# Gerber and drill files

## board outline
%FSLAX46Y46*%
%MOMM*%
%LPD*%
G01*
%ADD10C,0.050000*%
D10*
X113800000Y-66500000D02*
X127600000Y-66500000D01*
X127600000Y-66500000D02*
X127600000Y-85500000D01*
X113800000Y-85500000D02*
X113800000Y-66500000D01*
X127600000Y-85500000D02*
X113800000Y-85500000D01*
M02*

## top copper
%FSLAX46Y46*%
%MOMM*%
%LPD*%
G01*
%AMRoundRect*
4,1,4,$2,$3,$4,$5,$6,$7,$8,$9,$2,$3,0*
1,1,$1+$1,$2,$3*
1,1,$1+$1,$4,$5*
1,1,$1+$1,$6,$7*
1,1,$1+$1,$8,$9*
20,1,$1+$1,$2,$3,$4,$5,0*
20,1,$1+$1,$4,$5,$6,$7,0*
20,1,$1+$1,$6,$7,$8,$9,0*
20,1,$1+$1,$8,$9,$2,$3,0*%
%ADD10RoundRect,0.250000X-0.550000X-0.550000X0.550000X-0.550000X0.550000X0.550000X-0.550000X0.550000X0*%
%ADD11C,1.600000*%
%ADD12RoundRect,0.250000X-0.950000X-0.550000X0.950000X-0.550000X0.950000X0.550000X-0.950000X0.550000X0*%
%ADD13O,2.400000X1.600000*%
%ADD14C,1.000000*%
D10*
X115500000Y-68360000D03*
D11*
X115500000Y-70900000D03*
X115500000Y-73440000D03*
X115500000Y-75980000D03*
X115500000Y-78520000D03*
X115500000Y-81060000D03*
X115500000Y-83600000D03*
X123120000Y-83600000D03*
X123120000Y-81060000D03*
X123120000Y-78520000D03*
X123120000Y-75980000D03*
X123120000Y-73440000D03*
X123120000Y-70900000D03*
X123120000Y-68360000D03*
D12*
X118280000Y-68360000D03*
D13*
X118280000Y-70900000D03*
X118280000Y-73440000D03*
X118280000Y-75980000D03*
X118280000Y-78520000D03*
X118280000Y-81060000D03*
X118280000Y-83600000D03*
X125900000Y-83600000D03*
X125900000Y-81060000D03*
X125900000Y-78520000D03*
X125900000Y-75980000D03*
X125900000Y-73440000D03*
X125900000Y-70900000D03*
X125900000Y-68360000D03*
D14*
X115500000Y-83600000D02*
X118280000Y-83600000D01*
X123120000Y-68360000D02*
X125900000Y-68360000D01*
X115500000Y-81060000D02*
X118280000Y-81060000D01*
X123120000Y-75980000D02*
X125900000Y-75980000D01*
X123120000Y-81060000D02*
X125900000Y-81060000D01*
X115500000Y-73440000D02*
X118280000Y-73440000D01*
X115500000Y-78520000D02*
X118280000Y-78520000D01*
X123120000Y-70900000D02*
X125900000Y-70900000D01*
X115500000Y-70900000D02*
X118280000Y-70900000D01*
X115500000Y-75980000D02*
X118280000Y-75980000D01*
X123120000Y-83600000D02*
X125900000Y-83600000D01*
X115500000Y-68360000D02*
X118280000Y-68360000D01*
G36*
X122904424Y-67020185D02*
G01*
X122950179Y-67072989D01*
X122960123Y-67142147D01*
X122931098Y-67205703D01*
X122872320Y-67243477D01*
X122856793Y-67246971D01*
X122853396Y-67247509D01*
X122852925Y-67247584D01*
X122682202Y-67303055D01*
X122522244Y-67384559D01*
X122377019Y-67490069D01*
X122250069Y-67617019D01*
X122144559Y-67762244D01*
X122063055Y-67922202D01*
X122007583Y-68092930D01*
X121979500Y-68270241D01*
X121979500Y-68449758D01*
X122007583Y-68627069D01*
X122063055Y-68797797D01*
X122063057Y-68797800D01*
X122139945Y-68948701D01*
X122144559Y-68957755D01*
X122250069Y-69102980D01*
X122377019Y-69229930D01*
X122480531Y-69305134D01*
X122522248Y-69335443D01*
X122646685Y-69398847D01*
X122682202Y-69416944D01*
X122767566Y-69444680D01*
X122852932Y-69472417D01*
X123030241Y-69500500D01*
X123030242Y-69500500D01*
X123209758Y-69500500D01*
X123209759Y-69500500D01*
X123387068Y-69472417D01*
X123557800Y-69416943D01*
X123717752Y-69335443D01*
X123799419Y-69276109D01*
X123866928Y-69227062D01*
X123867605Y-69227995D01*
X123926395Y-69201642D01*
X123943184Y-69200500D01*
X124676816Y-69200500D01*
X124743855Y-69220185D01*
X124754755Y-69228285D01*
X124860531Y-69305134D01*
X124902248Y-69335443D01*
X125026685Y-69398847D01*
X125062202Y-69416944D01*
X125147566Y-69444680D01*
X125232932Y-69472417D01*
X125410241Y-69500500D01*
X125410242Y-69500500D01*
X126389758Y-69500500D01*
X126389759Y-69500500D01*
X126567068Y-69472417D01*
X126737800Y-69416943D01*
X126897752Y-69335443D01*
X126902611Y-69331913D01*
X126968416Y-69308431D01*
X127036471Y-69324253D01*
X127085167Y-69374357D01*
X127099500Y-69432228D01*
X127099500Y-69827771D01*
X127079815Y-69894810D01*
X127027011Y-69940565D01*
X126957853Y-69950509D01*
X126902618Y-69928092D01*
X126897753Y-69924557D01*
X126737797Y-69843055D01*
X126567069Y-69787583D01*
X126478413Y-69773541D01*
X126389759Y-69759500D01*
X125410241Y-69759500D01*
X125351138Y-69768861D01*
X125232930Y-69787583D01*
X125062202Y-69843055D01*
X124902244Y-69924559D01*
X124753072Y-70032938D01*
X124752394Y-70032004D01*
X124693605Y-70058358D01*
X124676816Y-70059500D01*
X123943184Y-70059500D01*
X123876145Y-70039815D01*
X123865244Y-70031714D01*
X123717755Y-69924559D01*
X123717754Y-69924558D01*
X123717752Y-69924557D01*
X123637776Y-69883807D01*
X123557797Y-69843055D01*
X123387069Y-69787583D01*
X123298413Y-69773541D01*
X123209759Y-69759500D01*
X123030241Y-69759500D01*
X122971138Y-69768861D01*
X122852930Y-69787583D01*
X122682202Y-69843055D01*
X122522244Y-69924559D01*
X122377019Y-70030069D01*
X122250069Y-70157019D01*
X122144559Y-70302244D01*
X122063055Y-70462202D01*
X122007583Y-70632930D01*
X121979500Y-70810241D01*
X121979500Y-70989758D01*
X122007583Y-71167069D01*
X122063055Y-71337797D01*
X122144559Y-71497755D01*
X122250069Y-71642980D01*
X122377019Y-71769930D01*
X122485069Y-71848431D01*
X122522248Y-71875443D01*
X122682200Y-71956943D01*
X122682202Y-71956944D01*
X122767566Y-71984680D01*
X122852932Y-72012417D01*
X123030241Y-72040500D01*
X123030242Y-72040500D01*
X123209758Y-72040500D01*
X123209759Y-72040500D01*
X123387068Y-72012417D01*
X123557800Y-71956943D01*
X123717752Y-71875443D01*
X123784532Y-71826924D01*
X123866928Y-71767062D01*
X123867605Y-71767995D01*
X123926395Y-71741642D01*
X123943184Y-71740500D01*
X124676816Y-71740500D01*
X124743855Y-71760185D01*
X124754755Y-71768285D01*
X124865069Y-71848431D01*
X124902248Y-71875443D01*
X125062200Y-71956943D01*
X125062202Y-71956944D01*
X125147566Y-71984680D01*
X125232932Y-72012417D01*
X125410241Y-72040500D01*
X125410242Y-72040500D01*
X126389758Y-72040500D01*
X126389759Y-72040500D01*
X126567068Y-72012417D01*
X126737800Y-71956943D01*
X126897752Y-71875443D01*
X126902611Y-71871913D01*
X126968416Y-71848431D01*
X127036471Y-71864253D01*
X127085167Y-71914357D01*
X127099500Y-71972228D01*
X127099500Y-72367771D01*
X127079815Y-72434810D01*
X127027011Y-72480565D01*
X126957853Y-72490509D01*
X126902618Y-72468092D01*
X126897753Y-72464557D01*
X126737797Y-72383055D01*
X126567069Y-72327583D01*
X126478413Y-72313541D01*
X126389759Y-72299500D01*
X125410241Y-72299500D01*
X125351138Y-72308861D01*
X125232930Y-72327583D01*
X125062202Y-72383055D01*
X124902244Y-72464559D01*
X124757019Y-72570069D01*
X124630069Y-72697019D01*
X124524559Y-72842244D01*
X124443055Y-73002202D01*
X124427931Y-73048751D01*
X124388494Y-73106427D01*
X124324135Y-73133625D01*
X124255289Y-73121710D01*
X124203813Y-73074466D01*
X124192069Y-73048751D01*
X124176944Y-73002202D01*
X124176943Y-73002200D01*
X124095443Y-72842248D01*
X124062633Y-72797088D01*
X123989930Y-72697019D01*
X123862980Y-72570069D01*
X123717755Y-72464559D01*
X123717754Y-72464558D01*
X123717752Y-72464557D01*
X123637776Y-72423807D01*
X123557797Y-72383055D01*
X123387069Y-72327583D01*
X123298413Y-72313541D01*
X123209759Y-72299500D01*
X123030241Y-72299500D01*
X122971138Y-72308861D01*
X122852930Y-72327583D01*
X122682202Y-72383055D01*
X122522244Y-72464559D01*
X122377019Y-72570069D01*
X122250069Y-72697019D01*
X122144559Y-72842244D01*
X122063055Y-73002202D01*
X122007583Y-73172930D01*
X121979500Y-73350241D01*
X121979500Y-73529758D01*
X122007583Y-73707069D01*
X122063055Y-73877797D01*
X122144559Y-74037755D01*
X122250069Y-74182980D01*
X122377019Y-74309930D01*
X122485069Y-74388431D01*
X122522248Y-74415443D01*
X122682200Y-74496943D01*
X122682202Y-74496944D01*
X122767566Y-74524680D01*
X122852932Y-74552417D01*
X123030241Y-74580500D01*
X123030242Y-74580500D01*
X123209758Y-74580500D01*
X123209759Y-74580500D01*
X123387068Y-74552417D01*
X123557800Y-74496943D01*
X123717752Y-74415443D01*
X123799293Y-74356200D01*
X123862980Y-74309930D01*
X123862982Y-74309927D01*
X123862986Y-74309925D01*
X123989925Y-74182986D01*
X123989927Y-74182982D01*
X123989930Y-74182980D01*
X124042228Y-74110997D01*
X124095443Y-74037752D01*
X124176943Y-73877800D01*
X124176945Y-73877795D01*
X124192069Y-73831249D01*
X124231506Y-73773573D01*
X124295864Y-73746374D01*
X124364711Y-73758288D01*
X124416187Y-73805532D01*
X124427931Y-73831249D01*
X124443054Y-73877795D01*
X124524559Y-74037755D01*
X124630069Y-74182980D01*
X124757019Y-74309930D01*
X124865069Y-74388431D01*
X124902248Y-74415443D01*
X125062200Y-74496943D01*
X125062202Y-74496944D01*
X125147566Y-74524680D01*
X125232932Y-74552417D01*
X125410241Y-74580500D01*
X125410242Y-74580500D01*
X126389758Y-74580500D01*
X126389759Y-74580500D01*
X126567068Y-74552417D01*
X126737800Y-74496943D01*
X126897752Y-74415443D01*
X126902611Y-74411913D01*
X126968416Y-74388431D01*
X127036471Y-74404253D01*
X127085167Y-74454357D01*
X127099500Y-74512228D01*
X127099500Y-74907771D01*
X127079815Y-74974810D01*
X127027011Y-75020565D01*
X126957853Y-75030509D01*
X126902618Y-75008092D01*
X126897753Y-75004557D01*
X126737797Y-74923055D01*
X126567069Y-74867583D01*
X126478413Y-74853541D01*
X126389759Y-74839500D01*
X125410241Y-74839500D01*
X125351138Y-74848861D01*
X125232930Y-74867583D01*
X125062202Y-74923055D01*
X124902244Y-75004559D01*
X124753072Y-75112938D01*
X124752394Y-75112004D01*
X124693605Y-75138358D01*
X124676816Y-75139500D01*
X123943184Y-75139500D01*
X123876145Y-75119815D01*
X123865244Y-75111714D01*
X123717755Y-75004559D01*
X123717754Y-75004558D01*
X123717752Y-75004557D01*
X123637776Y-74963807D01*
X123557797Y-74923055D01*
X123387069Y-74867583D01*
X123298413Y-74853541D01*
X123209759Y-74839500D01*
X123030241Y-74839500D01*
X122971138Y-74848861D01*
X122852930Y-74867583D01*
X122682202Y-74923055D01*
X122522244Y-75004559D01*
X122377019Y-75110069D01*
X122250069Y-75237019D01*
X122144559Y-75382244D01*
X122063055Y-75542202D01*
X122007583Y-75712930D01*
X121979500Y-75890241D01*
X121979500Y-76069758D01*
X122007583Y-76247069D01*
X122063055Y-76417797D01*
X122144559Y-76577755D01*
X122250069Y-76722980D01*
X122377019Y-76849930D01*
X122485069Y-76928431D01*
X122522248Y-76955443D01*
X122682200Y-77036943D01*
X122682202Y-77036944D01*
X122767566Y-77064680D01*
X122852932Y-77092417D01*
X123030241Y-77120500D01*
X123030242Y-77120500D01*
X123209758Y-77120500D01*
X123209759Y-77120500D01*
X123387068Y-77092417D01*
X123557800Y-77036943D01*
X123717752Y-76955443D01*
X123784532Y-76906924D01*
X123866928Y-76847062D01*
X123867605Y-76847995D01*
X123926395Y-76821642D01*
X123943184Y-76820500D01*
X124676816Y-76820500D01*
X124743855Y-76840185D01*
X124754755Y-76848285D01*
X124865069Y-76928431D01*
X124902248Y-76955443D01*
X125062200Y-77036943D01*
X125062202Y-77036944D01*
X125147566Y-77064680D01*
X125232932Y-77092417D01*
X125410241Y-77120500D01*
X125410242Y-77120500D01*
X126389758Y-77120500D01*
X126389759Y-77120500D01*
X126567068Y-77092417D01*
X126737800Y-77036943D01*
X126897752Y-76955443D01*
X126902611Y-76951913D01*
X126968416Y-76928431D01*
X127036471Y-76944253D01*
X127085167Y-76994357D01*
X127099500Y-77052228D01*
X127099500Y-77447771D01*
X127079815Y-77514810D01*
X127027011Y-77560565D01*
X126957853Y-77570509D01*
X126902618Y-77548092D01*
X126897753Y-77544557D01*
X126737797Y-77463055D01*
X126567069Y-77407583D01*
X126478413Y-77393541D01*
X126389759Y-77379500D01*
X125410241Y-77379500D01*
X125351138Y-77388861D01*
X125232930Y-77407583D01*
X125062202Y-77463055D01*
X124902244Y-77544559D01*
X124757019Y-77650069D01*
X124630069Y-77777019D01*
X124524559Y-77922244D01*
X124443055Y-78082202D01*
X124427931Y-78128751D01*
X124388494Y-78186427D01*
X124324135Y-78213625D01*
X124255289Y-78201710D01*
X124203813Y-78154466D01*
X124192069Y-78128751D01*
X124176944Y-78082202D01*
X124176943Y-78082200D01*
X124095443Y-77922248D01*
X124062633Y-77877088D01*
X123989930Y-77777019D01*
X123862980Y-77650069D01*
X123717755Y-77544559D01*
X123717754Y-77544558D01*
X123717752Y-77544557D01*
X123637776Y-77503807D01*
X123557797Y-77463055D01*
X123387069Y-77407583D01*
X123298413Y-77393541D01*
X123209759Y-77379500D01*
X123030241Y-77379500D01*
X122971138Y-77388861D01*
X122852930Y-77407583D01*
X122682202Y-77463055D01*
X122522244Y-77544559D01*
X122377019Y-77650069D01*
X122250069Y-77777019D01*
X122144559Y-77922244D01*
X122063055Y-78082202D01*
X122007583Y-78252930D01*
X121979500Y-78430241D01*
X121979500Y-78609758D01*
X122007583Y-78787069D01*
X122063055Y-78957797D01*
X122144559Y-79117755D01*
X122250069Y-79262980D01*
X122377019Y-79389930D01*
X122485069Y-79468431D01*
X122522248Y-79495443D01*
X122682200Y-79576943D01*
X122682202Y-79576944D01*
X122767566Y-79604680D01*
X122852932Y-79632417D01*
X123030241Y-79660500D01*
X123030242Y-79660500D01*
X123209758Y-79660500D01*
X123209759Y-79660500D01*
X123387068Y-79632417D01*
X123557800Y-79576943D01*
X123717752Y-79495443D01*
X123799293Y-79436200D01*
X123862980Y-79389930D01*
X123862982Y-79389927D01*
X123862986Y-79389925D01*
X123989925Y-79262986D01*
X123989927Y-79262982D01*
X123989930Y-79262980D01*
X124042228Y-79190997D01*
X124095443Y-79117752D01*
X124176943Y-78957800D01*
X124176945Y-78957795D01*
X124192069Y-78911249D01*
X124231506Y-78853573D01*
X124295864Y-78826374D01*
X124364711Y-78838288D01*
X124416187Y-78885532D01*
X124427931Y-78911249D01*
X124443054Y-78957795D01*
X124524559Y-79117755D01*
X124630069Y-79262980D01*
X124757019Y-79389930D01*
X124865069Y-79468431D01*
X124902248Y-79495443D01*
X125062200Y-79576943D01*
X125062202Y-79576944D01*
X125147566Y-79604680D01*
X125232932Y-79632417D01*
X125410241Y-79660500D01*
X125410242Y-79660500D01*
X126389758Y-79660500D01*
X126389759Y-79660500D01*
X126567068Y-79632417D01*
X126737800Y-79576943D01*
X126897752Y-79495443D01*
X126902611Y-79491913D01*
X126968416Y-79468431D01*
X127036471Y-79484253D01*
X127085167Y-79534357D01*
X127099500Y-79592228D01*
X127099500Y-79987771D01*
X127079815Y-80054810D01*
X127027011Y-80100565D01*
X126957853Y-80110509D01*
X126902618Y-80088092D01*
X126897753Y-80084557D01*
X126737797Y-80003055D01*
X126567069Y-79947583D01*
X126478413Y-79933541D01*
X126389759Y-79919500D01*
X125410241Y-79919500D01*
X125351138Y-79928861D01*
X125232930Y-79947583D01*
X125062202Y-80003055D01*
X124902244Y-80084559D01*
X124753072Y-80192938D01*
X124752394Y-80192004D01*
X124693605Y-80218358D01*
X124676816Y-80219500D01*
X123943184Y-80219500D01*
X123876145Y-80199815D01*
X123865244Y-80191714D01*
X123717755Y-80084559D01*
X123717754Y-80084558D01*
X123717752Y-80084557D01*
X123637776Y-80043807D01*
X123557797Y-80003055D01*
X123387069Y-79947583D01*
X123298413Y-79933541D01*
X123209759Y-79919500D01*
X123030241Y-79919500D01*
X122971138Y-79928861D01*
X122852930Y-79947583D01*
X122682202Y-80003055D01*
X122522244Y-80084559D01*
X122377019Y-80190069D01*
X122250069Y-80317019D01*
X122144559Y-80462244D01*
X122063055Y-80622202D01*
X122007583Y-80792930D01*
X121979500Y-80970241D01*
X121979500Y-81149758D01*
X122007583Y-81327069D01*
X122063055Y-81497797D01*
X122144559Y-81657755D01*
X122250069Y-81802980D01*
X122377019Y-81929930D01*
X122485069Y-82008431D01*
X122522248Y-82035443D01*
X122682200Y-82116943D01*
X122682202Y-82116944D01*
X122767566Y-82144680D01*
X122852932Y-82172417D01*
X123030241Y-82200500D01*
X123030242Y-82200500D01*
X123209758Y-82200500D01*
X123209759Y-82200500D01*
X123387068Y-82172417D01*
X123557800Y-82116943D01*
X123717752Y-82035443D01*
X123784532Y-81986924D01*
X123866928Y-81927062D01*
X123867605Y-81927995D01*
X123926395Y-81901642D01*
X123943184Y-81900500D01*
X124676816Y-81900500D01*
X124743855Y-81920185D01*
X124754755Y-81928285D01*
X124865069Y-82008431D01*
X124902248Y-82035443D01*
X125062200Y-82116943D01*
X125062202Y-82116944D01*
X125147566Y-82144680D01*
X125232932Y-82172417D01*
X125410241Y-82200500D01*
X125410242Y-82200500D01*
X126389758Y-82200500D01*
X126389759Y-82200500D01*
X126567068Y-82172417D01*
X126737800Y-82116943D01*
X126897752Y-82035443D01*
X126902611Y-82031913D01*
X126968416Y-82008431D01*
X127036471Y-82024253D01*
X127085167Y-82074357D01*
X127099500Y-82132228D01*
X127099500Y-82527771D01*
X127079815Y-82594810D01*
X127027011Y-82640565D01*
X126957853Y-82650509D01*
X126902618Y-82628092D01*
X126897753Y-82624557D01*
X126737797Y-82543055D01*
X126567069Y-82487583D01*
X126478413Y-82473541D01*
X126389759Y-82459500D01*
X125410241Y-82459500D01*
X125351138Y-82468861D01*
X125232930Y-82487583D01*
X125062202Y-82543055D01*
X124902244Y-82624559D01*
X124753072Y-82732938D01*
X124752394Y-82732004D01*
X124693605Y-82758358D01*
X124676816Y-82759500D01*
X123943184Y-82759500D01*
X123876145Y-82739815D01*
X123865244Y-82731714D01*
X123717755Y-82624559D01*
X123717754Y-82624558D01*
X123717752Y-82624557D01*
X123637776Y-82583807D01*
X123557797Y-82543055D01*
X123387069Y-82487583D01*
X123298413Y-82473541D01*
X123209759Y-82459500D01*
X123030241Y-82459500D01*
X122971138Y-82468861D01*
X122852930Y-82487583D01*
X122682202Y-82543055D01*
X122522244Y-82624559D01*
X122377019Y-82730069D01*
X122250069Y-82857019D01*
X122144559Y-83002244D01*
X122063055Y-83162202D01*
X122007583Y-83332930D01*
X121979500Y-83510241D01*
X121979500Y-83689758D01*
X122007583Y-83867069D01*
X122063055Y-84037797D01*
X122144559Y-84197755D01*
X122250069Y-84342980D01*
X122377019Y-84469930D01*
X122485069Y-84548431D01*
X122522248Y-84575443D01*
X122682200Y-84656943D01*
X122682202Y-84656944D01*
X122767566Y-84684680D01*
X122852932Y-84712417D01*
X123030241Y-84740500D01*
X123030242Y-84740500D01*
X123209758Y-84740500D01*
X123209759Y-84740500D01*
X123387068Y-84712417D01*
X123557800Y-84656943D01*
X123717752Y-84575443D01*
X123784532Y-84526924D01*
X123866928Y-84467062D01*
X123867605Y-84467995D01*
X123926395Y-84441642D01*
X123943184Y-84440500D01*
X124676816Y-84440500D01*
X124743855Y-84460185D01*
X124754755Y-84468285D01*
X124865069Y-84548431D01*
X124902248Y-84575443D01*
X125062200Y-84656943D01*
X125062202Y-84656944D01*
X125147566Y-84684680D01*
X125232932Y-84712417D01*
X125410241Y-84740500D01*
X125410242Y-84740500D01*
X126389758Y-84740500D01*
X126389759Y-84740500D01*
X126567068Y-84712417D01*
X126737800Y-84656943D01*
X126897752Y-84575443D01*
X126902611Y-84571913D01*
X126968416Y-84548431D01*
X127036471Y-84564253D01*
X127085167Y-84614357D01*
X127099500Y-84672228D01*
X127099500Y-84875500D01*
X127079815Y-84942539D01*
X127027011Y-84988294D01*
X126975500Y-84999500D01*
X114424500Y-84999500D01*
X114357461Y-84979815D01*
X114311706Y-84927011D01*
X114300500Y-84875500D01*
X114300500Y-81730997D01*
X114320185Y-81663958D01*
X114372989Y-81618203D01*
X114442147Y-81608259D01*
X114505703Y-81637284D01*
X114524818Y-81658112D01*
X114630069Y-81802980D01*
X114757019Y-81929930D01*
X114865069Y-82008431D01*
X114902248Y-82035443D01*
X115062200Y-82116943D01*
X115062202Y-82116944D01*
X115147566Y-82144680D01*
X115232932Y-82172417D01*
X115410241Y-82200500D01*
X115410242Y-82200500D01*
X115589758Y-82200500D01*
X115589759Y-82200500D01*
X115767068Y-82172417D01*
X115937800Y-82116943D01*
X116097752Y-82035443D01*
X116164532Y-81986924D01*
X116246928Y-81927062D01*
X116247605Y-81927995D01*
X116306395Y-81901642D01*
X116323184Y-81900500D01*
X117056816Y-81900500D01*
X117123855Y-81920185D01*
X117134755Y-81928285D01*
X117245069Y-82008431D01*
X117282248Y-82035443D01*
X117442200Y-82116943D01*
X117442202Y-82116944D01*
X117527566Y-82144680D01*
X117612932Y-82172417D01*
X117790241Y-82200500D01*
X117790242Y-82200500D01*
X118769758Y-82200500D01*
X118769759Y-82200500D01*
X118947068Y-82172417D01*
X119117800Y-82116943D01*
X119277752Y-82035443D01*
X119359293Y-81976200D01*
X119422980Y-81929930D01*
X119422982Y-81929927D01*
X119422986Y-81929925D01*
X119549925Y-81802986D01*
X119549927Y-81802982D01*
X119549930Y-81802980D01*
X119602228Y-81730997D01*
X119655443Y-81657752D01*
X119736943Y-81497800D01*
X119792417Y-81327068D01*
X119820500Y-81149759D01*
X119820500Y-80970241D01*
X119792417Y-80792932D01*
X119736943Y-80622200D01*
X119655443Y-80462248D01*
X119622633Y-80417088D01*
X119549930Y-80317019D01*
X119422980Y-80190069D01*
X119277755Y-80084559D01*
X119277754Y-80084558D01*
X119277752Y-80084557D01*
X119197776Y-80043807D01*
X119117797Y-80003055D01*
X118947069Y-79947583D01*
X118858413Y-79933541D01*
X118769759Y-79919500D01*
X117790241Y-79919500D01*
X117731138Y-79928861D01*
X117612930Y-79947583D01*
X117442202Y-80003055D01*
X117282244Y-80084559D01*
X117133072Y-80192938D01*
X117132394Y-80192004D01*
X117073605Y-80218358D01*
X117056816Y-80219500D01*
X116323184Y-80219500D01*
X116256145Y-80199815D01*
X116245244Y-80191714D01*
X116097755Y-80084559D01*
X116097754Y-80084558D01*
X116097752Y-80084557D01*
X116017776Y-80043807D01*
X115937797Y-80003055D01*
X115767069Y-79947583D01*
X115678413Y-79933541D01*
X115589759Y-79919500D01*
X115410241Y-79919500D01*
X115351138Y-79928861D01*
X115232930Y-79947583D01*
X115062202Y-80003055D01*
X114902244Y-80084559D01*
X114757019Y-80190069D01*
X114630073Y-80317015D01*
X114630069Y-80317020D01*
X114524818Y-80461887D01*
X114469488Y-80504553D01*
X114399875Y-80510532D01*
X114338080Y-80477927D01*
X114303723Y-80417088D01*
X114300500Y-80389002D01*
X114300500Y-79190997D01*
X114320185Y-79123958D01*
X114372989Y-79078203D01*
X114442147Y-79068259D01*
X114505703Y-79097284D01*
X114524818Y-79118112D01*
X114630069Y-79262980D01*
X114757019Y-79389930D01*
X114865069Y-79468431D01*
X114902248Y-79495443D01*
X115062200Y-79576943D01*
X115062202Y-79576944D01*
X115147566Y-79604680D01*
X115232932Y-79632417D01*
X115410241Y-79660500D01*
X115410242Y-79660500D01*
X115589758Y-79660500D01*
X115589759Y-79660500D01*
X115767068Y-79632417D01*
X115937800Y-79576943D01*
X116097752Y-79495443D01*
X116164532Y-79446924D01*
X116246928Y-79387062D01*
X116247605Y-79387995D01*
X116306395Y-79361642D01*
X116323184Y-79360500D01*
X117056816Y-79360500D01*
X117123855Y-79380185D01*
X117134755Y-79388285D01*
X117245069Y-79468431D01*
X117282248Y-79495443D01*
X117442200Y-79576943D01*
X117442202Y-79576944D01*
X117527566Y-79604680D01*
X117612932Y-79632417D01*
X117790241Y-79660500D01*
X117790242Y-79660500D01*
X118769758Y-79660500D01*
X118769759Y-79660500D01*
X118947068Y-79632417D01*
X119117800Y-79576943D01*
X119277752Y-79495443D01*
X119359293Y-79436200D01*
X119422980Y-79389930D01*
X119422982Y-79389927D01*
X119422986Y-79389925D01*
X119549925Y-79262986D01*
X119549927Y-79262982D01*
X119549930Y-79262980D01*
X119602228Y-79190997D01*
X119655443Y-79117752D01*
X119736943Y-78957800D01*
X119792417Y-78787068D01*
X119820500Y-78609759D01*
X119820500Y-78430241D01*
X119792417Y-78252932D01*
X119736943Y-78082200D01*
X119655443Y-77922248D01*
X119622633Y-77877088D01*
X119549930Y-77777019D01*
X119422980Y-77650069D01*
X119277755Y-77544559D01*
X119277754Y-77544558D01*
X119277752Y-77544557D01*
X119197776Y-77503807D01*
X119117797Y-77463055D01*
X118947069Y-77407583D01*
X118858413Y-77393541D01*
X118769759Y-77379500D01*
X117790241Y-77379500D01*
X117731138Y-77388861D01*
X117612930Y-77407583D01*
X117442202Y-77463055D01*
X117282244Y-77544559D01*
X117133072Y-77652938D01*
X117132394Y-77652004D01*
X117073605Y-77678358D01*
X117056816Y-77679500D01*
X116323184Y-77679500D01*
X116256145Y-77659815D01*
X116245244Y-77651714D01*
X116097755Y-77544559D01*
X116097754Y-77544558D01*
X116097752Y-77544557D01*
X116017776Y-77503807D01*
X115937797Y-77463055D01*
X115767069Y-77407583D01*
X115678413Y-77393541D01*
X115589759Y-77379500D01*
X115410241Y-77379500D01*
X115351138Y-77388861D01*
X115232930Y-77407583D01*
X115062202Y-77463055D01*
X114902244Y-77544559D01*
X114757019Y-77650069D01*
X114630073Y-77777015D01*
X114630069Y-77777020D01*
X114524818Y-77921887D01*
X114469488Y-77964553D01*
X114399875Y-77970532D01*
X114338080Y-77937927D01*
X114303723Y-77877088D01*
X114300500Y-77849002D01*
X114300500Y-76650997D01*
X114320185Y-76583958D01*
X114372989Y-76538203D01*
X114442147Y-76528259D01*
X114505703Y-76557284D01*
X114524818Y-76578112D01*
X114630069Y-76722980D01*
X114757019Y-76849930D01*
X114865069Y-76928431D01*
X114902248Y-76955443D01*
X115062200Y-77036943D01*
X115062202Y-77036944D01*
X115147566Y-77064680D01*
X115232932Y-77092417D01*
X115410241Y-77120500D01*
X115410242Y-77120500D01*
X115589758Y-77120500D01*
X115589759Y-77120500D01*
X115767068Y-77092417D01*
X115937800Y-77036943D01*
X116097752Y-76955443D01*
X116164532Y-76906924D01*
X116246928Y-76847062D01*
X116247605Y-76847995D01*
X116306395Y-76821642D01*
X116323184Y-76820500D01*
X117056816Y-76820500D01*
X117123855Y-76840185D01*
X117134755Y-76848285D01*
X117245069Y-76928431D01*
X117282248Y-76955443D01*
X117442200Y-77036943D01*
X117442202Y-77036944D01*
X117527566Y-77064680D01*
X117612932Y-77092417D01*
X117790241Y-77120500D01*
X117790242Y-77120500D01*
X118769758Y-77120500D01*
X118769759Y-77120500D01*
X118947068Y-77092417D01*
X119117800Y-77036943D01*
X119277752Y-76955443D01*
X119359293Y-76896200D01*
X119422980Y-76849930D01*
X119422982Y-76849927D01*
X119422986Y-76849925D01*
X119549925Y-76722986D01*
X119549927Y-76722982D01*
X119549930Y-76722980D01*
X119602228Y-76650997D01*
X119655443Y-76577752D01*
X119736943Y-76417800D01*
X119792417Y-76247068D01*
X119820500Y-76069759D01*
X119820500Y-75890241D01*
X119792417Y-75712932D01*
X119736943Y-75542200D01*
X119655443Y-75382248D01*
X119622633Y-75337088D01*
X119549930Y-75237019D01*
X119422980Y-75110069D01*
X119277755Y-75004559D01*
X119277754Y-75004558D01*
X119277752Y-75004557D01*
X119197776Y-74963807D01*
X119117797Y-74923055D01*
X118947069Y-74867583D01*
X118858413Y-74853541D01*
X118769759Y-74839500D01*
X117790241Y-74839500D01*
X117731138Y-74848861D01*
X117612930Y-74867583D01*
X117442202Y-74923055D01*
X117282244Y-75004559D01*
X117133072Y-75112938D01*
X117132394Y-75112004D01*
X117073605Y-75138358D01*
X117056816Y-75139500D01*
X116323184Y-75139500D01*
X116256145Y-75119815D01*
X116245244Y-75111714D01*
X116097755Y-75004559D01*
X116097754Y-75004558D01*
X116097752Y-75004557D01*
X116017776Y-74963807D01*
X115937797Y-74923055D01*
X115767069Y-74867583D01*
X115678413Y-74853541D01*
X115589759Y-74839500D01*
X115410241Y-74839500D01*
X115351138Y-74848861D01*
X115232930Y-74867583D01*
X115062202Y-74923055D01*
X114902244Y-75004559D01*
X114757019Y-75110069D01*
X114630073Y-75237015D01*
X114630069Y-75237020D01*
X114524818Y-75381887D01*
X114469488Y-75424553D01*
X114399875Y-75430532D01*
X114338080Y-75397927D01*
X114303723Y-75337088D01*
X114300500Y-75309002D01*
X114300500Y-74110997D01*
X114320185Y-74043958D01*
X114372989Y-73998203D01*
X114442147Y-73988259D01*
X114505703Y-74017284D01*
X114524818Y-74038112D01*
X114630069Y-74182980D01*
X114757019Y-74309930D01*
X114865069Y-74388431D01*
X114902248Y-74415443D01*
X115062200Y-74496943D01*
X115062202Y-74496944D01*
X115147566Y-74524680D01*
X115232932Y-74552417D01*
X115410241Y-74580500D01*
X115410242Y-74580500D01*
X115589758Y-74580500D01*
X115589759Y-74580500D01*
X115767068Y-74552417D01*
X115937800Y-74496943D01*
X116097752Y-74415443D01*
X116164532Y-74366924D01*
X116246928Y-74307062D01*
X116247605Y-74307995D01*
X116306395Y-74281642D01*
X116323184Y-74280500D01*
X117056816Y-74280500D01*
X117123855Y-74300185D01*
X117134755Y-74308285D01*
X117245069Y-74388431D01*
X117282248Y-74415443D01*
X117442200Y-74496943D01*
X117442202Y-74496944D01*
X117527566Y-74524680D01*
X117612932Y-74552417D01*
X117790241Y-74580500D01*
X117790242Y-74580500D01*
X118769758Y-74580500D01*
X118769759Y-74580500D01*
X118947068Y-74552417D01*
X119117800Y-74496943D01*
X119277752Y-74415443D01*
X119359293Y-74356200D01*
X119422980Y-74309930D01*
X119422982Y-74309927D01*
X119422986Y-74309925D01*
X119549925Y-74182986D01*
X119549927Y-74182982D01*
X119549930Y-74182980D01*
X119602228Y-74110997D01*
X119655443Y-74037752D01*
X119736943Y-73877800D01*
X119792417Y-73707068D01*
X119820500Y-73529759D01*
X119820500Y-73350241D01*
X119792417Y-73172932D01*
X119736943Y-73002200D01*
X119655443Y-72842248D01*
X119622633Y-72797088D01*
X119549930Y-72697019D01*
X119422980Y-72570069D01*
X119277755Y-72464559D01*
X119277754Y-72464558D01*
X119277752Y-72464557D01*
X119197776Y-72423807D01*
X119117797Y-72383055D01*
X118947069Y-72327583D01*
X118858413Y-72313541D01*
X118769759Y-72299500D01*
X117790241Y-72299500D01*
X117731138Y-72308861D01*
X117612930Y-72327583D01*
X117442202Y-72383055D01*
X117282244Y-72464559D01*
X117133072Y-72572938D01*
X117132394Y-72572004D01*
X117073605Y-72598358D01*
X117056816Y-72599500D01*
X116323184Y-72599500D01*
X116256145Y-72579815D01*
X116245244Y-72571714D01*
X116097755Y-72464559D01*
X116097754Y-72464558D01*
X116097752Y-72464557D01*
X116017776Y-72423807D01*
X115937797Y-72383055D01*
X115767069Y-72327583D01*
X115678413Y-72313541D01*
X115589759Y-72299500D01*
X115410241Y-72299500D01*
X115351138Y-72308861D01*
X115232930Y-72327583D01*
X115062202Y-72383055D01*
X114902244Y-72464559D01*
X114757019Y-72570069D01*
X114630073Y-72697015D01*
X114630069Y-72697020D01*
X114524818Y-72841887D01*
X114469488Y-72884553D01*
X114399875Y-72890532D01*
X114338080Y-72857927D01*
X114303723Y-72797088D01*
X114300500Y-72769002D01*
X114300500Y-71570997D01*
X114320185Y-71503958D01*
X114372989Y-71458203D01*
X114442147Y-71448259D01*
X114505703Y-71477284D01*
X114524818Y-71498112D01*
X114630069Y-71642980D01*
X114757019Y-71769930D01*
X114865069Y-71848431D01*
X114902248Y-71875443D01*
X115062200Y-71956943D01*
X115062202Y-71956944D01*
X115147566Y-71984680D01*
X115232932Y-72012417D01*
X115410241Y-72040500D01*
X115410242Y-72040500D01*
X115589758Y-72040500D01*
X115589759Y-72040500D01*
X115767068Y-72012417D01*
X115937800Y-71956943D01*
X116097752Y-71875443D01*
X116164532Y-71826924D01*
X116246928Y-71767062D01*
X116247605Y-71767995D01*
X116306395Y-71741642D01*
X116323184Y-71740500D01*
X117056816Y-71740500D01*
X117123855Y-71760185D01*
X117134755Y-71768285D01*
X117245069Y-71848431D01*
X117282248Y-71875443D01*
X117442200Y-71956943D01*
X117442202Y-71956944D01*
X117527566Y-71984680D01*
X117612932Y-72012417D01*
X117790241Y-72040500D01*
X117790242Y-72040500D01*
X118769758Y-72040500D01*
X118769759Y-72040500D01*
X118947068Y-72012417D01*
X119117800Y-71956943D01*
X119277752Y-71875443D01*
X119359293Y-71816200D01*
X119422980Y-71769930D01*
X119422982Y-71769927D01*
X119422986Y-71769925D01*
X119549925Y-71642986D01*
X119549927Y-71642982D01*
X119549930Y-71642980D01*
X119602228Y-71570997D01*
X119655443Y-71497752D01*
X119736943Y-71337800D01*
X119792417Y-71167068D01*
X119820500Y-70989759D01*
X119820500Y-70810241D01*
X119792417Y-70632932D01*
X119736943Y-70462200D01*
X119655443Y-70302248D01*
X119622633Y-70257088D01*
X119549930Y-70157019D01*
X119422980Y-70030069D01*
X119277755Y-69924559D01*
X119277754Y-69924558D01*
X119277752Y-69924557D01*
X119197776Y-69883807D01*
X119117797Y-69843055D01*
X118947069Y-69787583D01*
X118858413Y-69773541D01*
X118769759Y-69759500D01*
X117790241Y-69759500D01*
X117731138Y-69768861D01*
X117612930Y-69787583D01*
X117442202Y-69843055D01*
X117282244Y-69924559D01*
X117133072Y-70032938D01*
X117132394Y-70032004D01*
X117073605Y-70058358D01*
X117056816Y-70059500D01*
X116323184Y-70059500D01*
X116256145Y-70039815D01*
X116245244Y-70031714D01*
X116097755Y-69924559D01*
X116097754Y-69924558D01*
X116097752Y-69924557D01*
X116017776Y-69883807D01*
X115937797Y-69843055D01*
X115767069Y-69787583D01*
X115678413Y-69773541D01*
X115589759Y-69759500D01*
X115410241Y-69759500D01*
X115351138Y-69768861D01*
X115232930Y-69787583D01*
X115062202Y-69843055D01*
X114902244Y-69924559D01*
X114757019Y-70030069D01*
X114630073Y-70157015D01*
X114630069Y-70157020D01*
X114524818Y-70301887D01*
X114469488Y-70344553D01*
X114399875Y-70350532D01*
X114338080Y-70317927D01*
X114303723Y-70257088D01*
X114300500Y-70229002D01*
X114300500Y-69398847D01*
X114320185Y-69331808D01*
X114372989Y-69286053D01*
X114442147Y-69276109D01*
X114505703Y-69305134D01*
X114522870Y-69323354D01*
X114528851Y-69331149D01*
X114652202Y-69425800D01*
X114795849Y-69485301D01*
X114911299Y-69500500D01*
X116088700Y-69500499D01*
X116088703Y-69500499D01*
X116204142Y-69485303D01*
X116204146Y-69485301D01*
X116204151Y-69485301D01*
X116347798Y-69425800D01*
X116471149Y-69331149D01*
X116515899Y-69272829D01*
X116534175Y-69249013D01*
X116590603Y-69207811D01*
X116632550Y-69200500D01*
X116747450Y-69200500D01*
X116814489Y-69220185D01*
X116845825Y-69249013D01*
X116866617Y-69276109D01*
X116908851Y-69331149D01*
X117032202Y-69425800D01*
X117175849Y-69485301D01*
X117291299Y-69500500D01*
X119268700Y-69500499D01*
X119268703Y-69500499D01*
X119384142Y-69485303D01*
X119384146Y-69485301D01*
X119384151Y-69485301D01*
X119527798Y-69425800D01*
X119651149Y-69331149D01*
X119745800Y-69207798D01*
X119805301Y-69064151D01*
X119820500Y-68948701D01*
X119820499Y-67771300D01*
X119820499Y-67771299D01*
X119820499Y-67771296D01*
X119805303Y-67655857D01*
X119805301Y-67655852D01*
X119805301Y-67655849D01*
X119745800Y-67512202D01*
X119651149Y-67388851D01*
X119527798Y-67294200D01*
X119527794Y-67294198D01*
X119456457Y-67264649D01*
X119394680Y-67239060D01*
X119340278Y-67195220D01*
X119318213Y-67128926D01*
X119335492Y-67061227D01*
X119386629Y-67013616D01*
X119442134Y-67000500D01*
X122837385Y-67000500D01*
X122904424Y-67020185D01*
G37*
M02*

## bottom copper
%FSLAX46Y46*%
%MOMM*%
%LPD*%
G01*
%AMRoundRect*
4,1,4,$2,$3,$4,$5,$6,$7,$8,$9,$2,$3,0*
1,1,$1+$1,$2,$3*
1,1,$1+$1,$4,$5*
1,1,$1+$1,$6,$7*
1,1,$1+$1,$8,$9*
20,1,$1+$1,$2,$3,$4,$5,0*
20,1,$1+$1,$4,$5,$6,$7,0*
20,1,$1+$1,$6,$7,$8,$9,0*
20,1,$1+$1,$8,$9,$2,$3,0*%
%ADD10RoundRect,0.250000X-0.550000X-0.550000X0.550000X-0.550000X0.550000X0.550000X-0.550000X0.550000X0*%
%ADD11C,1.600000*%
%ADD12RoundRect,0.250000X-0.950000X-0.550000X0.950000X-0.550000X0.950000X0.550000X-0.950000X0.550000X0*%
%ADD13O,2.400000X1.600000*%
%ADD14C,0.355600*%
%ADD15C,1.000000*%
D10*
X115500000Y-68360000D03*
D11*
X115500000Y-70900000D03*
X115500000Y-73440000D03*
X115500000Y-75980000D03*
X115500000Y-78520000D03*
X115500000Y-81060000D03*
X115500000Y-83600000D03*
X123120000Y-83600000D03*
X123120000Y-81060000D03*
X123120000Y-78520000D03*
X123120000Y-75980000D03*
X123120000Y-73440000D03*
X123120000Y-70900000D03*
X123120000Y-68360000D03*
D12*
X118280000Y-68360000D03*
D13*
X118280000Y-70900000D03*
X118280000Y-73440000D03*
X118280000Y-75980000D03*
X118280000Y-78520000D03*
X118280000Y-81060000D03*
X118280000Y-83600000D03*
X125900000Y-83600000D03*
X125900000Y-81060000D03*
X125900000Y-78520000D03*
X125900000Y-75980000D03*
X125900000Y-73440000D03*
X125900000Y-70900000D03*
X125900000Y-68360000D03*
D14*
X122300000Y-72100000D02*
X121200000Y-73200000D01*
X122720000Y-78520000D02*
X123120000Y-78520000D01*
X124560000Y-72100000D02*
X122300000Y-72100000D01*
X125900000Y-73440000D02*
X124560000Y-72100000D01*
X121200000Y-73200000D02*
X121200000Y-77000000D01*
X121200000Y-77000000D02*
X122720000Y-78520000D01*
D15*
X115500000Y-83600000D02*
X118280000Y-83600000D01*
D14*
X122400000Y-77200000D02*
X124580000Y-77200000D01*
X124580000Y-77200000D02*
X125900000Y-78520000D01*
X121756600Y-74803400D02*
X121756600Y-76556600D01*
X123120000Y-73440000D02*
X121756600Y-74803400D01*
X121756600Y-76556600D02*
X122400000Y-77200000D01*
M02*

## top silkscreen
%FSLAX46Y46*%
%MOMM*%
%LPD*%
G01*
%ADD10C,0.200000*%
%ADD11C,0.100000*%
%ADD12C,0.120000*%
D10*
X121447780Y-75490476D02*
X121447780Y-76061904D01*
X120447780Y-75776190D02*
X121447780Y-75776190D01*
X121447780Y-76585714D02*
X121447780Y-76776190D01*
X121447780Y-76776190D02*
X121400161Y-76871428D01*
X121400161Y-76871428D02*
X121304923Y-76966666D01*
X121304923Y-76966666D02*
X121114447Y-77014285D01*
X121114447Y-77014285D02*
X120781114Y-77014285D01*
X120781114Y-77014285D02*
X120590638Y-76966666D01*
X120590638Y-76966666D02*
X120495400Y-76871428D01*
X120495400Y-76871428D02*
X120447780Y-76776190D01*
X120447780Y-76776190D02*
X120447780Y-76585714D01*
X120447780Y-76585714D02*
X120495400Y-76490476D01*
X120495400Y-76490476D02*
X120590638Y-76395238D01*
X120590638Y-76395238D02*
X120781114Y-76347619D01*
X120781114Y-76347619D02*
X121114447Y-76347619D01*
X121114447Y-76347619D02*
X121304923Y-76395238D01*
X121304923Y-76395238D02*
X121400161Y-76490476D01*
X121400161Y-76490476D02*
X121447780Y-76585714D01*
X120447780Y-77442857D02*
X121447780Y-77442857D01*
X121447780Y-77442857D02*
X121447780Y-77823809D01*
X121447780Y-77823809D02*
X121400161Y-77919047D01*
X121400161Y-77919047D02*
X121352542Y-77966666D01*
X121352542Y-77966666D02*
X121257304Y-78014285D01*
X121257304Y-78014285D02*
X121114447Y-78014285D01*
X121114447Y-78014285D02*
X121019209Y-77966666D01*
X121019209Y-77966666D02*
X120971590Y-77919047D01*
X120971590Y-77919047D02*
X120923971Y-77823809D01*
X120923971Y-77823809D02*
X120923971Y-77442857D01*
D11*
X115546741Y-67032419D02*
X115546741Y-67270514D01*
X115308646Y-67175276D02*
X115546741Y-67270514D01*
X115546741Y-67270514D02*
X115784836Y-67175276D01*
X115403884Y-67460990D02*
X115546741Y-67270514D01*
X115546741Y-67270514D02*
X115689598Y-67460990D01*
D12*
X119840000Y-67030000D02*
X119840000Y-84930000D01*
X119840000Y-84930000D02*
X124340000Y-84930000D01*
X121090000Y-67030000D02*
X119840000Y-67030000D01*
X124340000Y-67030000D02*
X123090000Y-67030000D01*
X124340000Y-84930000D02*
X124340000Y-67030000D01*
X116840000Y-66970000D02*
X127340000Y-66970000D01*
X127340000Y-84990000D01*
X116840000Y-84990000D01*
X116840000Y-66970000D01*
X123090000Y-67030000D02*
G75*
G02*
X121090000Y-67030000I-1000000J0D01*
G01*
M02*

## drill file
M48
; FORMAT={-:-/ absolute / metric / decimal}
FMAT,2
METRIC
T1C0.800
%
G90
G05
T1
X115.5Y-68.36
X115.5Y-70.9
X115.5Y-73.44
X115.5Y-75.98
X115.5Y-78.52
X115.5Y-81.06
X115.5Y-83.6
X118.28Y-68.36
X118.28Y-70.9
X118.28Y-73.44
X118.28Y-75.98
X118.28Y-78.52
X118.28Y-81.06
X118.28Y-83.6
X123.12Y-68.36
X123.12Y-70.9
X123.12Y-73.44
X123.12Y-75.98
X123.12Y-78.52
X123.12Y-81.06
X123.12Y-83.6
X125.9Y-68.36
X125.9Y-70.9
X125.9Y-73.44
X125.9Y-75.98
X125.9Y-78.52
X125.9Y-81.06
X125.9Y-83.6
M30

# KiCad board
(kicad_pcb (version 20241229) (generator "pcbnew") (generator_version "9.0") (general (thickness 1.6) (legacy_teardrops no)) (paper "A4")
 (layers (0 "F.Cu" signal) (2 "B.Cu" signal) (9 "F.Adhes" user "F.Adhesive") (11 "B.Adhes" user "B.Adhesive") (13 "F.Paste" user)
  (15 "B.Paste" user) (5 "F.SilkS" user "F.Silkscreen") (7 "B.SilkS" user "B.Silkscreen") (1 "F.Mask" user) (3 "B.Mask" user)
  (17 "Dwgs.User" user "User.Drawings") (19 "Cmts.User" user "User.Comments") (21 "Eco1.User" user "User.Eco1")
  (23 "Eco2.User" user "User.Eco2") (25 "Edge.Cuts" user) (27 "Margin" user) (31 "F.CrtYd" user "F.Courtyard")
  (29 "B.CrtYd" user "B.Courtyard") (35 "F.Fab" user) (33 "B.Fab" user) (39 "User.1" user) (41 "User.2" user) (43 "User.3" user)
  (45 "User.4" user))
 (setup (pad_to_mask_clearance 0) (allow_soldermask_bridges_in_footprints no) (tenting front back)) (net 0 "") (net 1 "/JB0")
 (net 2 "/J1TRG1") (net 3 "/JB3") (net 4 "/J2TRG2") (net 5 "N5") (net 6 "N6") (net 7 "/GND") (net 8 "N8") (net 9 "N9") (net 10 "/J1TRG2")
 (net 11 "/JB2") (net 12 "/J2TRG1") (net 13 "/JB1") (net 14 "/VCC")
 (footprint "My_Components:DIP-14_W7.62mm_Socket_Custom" (layer "F.Cu") (at 115.5 68.36)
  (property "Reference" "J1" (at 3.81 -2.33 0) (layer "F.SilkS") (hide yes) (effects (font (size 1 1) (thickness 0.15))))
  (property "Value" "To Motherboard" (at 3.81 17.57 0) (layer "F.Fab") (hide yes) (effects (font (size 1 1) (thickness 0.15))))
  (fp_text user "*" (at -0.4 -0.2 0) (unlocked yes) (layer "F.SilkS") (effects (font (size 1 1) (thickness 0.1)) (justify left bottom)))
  (pad "1" thru_hole roundrect (at 0 0) (size 1.6 1.6) (drill 0.8) (layers "*.Cu" "*.Mask") (remove_unused_layers no)
   (roundrect_rratio 0.15625) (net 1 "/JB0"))
  (pad "2" thru_hole circle (at 0 2.54) (size 1.6 1.6) (drill 0.8) (layers "*.Cu" "*.Mask") (remove_unused_layers no) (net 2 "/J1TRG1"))
  (pad "3" thru_hole circle (at 0 5.08) (size 1.6 1.6) (drill 0.8) (layers "*.Cu" "*.Mask") (remove_unused_layers no) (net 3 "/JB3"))
  (pad "4" thru_hole circle (at 0 7.62) (size 1.6 1.6) (drill 0.8) (layers "*.Cu" "*.Mask") (remove_unused_layers no) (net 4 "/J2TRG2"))
  (pad "5" thru_hole circle (at 0 10.16) (size 1.6 1.6) (drill 0.8) (layers "*.Cu" "*.Mask") (remove_unused_layers no) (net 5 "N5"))
  (pad "6" thru_hole circle (at 0 12.7) (size 1.6 1.6) (drill 0.8) (layers "*.Cu" "*.Mask") (remove_unused_layers no) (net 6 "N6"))
  (pad "7" thru_hole circle (at 0 15.24) (size 1.6 1.6) (drill 0.8) (layers "*.Cu" "*.Mask") (remove_unused_layers no) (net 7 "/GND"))
  (pad "8" thru_hole circle (at 7.62 15.24) (size 1.6 1.6) (drill 0.8) (layers "*.Cu" "*.Mask") (remove_unused_layers no) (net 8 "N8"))
  (pad "9" thru_hole circle (at 7.62 12.7) (size 1.6 1.6) (drill 0.8) (layers "*.Cu" "*.Mask") (remove_unused_layers no) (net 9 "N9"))
  (pad "10" thru_hole circle (at 7.62 10.16) (size 1.6 1.6) (drill 0.8) (layers "*.Cu" "*.Mask") (remove_unused_layers no)
   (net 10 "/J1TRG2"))
  (pad "11" thru_hole circle (at 7.62 7.62) (size 1.6 1.6) (drill 0.8) (layers "*.Cu" "*.Mask") (remove_unused_layers no) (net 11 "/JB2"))
  (pad "12" thru_hole circle (at 7.62 5.08) (size 1.6 1.6) (drill 0.8) (layers "*.Cu" "*.Mask") (remove_unused_layers no) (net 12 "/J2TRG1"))
  (pad "13" thru_hole circle (at 7.62 2.54) (size 1.6 1.6) (drill 0.8) (layers "*.Cu" "*.Mask") (remove_unused_layers no) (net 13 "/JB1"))
  (pad "14" thru_hole circle (at 7.62 0) (size 1.6 1.6) (drill 0.8) (layers "*.Cu" "*.Mask") (remove_unused_layers no) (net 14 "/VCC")))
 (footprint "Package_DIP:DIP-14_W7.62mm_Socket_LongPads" (layer "F.Cu") (at 118.28 68.36)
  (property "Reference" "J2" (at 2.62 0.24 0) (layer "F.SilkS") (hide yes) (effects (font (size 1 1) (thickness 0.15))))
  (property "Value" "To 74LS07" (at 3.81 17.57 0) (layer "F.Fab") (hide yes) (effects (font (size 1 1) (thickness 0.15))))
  (fp_line (start 1.56 -1.33) (end 1.56 16.57) (stroke (width 0.12) (type solid)) (layer "F.SilkS"))
  (fp_line (start 1.56 16.57) (end 6.06 16.57) (stroke (width 0.12) (type solid)) (layer "F.SilkS"))
  (fp_line (start 2.81 -1.33) (end 1.56 -1.33) (stroke (width 0.12) (type solid)) (layer "F.SilkS"))
  (fp_line (start 6.06 -1.33) (end 4.81 -1.33) (stroke (width 0.12) (type solid)) (layer "F.SilkS"))
  (fp_line (start 6.06 16.57) (end 6.06 -1.33) (stroke (width 0.12) (type solid)) (layer "F.SilkS"))
  (fp_rect (start -1.44 -1.39) (end 9.06 16.63) (stroke (width 0.12) (type solid)) (fill no) (layer "F.SilkS"))
  (fp_arc (start 4.81 -1.33) (mid 3.81 -0.33) (end 2.81 -1.33) (stroke (width 0.12) (type solid)) (layer "F.SilkS"))
  (pad "1" thru_hole roundrect (at 0 0) (size 2.4 1.6) (drill 0.8) (layers "*.Cu" "*.Mask") (remove_unused_layers no)
   (roundrect_rratio 0.15625) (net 1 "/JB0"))
  (pad "2" thru_hole oval (at 0 2.54) (size 2.4 1.6) (drill 0.8) (layers "*.Cu" "*.Mask") (remove_unused_layers no) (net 2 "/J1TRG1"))
  (pad "3" thru_hole oval (at 0 5.08) (size 2.4 1.6) (drill 0.8) (layers "*.Cu" "*.Mask") (remove_unused_layers no) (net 3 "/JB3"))
  (pad "4" thru_hole oval (at 0 7.62) (size 2.4 1.6) (drill 0.8) (layers "*.Cu" "*.Mask") (remove_unused_layers no) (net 4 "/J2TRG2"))
  (pad "5" thru_hole oval (at 0 10.16) (size 2.4 1.6) (drill 0.8) (layers "*.Cu" "*.Mask") (remove_unused_layers no) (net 5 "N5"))
  (pad "6" thru_hole oval (at 0 12.7) (size 2.4 1.6) (drill 0.8) (layers "*.Cu" "*.Mask") (remove_unused_layers no) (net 6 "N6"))
  (pad "7" thru_hole oval (at 0 15.24) (size 2.4 1.6) (drill 0.8) (layers "*.Cu" "*.Mask") (remove_unused_layers no) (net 7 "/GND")
   (thermal_bridge_angle 45))
  (pad "8" thru_hole oval (at 7.62 15.24) (size 2.4 1.6) (drill 0.8) (layers "*.Cu" "*.Mask") (remove_unused_layers no) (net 8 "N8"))
  (pad "9" thru_hole oval (at 7.62 12.7) (size 2.4 1.6) (drill 0.8) (layers "*.Cu" "*.Mask") (remove_unused_layers no) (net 9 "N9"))
  (pad "10" thru_hole oval (at 7.62 10.16) (size 2.4 1.6) (drill 0.8) (layers "*.Cu" "*.Mask") (remove_unused_layers no) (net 12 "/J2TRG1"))
  (pad "11" thru_hole oval (at 7.62 7.62) (size 2.4 1.6) (drill 0.8) (layers "*.Cu" "*.Mask") (remove_unused_layers no) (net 11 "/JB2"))
  (pad "12" thru_hole oval (at 7.62 5.08) (size 2.4 1.6) (drill 0.8) (layers "*.Cu" "*.Mask") (remove_unused_layers no) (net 10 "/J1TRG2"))
  (pad "13" thru_hole oval (at 7.62 2.54) (size 2.4 1.6) (drill 0.8) (layers "*.Cu" "*.Mask") (remove_unused_layers no) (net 13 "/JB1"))
  (pad "14" thru_hole oval (at 7.62 0) (size 2.4 1.6) (drill 0.8) (layers "*.Cu" "*.Mask") (remove_unused_layers no) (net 14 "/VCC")))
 (gr_line (start 113.8 66.5) (end 127.6 66.5) (stroke (width 0.05) (type default)) (layer "Edge.Cuts"))
 (gr_line (start 127.6 66.5) (end 127.6 85.5) (stroke (width 0.05) (type solid)) (layer "Edge.Cuts"))
 (gr_line (start 113.8 85.5) (end 113.8 66.5) (stroke (width 0.05) (type solid)) (layer "Edge.Cuts"))
 (gr_line (start 127.6 85.5) (end 113.8 85.5) (stroke (width 0.05) (type default)) (layer "Edge.Cuts"))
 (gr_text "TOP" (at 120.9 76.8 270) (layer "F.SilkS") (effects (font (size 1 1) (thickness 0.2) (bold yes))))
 (segment (start 122.3 72.1) (end 121.2 73.2) (width 0.3556) (layer "B.Cu") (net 10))
 (segment (start 122.72 78.52) (end 123.12 78.52) (width 0.3556) (layer "B.Cu") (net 10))
 (segment (start 124.56 72.1) (end 122.3 72.1) (width 0.3556) (layer "B.Cu") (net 10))
 (segment (start 125.9 73.44) (end 124.56 72.1) (width 0.3556) (layer "B.Cu") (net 10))
 (segment (start 121.2 73.2) (end 121.2 77) (width 0.3556) (layer "B.Cu") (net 10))
 (segment (start 121.2 77) (end 122.72 78.52) (width 0.3556) (layer "B.Cu") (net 10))
 (segment (start 115.5 83.6) (end 118.28 83.6) (width 1) (layer "F.Cu") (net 7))
 (segment (start 115.5 83.6) (end 118.28 83.6) (width 1) (layer "B.Cu") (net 7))
 (segment (start 123.12 68.36) (end 125.9 68.36) (width 1) (layer "F.Cu") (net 14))
 (segment (start 115.5 81.06) (end 118.28 81.06) (width 1) (layer "F.Cu") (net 6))
 (segment (start 123.12 75.98) (end 125.9 75.98) (width 1) (layer "F.Cu") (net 11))
 (segment (start 123.12 81.06) (end 125.9 81.06) (width 1) (layer "F.Cu") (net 9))
 (segment (start 115.5 73.44) (end 118.28 73.44) (width 1) (layer "F.Cu") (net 3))
 (segment (start 115.5 78.52) (end 118.28 78.52) (width 1) (layer "F.Cu") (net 5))
 (segment (start 123.12 70.9) (end 125.9 70.9) (width 1) (layer "F.Cu") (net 13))
 (segment (start 115.5 70.9) (end 118.28 70.9) (width 1) (layer "F.Cu") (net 2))
 (segment (start 115.5 75.98) (end 118.28 75.98) (width 1) (layer "F.Cu") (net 4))
 (segment (start 122.4 77.2) (end 124.58 77.2) (width 0.3556) (layer "B.Cu") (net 12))
 (segment (start 124.58 77.2) (end 125.9 78.52) (width 0.3556) (layer "B.Cu") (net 12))
 (segment (start 121.7566 74.8034) (end 121.7566 76.5566) (width 0.3556) (layer "B.Cu") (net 12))
 (segment (start 123.12 73.44) (end 121.7566 74.8034) (width 0.3556) (layer "B.Cu") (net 12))
 (segment (start 121.7566 76.5566) (end 122.4 77.2) (width 0.3556) (layer "B.Cu") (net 12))
 (segment (start 123.12 83.6) (end 125.9 83.6) (width 1) (layer "F.Cu") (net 8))
 (segment (start 115.5 68.36) (end 118.28 68.36) (width 1) (layer "F.Cu") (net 1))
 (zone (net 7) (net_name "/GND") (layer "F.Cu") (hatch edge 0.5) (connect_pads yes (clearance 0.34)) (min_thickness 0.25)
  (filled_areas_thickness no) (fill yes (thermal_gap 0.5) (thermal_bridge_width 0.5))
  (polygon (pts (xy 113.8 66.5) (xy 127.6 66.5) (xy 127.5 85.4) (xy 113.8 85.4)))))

